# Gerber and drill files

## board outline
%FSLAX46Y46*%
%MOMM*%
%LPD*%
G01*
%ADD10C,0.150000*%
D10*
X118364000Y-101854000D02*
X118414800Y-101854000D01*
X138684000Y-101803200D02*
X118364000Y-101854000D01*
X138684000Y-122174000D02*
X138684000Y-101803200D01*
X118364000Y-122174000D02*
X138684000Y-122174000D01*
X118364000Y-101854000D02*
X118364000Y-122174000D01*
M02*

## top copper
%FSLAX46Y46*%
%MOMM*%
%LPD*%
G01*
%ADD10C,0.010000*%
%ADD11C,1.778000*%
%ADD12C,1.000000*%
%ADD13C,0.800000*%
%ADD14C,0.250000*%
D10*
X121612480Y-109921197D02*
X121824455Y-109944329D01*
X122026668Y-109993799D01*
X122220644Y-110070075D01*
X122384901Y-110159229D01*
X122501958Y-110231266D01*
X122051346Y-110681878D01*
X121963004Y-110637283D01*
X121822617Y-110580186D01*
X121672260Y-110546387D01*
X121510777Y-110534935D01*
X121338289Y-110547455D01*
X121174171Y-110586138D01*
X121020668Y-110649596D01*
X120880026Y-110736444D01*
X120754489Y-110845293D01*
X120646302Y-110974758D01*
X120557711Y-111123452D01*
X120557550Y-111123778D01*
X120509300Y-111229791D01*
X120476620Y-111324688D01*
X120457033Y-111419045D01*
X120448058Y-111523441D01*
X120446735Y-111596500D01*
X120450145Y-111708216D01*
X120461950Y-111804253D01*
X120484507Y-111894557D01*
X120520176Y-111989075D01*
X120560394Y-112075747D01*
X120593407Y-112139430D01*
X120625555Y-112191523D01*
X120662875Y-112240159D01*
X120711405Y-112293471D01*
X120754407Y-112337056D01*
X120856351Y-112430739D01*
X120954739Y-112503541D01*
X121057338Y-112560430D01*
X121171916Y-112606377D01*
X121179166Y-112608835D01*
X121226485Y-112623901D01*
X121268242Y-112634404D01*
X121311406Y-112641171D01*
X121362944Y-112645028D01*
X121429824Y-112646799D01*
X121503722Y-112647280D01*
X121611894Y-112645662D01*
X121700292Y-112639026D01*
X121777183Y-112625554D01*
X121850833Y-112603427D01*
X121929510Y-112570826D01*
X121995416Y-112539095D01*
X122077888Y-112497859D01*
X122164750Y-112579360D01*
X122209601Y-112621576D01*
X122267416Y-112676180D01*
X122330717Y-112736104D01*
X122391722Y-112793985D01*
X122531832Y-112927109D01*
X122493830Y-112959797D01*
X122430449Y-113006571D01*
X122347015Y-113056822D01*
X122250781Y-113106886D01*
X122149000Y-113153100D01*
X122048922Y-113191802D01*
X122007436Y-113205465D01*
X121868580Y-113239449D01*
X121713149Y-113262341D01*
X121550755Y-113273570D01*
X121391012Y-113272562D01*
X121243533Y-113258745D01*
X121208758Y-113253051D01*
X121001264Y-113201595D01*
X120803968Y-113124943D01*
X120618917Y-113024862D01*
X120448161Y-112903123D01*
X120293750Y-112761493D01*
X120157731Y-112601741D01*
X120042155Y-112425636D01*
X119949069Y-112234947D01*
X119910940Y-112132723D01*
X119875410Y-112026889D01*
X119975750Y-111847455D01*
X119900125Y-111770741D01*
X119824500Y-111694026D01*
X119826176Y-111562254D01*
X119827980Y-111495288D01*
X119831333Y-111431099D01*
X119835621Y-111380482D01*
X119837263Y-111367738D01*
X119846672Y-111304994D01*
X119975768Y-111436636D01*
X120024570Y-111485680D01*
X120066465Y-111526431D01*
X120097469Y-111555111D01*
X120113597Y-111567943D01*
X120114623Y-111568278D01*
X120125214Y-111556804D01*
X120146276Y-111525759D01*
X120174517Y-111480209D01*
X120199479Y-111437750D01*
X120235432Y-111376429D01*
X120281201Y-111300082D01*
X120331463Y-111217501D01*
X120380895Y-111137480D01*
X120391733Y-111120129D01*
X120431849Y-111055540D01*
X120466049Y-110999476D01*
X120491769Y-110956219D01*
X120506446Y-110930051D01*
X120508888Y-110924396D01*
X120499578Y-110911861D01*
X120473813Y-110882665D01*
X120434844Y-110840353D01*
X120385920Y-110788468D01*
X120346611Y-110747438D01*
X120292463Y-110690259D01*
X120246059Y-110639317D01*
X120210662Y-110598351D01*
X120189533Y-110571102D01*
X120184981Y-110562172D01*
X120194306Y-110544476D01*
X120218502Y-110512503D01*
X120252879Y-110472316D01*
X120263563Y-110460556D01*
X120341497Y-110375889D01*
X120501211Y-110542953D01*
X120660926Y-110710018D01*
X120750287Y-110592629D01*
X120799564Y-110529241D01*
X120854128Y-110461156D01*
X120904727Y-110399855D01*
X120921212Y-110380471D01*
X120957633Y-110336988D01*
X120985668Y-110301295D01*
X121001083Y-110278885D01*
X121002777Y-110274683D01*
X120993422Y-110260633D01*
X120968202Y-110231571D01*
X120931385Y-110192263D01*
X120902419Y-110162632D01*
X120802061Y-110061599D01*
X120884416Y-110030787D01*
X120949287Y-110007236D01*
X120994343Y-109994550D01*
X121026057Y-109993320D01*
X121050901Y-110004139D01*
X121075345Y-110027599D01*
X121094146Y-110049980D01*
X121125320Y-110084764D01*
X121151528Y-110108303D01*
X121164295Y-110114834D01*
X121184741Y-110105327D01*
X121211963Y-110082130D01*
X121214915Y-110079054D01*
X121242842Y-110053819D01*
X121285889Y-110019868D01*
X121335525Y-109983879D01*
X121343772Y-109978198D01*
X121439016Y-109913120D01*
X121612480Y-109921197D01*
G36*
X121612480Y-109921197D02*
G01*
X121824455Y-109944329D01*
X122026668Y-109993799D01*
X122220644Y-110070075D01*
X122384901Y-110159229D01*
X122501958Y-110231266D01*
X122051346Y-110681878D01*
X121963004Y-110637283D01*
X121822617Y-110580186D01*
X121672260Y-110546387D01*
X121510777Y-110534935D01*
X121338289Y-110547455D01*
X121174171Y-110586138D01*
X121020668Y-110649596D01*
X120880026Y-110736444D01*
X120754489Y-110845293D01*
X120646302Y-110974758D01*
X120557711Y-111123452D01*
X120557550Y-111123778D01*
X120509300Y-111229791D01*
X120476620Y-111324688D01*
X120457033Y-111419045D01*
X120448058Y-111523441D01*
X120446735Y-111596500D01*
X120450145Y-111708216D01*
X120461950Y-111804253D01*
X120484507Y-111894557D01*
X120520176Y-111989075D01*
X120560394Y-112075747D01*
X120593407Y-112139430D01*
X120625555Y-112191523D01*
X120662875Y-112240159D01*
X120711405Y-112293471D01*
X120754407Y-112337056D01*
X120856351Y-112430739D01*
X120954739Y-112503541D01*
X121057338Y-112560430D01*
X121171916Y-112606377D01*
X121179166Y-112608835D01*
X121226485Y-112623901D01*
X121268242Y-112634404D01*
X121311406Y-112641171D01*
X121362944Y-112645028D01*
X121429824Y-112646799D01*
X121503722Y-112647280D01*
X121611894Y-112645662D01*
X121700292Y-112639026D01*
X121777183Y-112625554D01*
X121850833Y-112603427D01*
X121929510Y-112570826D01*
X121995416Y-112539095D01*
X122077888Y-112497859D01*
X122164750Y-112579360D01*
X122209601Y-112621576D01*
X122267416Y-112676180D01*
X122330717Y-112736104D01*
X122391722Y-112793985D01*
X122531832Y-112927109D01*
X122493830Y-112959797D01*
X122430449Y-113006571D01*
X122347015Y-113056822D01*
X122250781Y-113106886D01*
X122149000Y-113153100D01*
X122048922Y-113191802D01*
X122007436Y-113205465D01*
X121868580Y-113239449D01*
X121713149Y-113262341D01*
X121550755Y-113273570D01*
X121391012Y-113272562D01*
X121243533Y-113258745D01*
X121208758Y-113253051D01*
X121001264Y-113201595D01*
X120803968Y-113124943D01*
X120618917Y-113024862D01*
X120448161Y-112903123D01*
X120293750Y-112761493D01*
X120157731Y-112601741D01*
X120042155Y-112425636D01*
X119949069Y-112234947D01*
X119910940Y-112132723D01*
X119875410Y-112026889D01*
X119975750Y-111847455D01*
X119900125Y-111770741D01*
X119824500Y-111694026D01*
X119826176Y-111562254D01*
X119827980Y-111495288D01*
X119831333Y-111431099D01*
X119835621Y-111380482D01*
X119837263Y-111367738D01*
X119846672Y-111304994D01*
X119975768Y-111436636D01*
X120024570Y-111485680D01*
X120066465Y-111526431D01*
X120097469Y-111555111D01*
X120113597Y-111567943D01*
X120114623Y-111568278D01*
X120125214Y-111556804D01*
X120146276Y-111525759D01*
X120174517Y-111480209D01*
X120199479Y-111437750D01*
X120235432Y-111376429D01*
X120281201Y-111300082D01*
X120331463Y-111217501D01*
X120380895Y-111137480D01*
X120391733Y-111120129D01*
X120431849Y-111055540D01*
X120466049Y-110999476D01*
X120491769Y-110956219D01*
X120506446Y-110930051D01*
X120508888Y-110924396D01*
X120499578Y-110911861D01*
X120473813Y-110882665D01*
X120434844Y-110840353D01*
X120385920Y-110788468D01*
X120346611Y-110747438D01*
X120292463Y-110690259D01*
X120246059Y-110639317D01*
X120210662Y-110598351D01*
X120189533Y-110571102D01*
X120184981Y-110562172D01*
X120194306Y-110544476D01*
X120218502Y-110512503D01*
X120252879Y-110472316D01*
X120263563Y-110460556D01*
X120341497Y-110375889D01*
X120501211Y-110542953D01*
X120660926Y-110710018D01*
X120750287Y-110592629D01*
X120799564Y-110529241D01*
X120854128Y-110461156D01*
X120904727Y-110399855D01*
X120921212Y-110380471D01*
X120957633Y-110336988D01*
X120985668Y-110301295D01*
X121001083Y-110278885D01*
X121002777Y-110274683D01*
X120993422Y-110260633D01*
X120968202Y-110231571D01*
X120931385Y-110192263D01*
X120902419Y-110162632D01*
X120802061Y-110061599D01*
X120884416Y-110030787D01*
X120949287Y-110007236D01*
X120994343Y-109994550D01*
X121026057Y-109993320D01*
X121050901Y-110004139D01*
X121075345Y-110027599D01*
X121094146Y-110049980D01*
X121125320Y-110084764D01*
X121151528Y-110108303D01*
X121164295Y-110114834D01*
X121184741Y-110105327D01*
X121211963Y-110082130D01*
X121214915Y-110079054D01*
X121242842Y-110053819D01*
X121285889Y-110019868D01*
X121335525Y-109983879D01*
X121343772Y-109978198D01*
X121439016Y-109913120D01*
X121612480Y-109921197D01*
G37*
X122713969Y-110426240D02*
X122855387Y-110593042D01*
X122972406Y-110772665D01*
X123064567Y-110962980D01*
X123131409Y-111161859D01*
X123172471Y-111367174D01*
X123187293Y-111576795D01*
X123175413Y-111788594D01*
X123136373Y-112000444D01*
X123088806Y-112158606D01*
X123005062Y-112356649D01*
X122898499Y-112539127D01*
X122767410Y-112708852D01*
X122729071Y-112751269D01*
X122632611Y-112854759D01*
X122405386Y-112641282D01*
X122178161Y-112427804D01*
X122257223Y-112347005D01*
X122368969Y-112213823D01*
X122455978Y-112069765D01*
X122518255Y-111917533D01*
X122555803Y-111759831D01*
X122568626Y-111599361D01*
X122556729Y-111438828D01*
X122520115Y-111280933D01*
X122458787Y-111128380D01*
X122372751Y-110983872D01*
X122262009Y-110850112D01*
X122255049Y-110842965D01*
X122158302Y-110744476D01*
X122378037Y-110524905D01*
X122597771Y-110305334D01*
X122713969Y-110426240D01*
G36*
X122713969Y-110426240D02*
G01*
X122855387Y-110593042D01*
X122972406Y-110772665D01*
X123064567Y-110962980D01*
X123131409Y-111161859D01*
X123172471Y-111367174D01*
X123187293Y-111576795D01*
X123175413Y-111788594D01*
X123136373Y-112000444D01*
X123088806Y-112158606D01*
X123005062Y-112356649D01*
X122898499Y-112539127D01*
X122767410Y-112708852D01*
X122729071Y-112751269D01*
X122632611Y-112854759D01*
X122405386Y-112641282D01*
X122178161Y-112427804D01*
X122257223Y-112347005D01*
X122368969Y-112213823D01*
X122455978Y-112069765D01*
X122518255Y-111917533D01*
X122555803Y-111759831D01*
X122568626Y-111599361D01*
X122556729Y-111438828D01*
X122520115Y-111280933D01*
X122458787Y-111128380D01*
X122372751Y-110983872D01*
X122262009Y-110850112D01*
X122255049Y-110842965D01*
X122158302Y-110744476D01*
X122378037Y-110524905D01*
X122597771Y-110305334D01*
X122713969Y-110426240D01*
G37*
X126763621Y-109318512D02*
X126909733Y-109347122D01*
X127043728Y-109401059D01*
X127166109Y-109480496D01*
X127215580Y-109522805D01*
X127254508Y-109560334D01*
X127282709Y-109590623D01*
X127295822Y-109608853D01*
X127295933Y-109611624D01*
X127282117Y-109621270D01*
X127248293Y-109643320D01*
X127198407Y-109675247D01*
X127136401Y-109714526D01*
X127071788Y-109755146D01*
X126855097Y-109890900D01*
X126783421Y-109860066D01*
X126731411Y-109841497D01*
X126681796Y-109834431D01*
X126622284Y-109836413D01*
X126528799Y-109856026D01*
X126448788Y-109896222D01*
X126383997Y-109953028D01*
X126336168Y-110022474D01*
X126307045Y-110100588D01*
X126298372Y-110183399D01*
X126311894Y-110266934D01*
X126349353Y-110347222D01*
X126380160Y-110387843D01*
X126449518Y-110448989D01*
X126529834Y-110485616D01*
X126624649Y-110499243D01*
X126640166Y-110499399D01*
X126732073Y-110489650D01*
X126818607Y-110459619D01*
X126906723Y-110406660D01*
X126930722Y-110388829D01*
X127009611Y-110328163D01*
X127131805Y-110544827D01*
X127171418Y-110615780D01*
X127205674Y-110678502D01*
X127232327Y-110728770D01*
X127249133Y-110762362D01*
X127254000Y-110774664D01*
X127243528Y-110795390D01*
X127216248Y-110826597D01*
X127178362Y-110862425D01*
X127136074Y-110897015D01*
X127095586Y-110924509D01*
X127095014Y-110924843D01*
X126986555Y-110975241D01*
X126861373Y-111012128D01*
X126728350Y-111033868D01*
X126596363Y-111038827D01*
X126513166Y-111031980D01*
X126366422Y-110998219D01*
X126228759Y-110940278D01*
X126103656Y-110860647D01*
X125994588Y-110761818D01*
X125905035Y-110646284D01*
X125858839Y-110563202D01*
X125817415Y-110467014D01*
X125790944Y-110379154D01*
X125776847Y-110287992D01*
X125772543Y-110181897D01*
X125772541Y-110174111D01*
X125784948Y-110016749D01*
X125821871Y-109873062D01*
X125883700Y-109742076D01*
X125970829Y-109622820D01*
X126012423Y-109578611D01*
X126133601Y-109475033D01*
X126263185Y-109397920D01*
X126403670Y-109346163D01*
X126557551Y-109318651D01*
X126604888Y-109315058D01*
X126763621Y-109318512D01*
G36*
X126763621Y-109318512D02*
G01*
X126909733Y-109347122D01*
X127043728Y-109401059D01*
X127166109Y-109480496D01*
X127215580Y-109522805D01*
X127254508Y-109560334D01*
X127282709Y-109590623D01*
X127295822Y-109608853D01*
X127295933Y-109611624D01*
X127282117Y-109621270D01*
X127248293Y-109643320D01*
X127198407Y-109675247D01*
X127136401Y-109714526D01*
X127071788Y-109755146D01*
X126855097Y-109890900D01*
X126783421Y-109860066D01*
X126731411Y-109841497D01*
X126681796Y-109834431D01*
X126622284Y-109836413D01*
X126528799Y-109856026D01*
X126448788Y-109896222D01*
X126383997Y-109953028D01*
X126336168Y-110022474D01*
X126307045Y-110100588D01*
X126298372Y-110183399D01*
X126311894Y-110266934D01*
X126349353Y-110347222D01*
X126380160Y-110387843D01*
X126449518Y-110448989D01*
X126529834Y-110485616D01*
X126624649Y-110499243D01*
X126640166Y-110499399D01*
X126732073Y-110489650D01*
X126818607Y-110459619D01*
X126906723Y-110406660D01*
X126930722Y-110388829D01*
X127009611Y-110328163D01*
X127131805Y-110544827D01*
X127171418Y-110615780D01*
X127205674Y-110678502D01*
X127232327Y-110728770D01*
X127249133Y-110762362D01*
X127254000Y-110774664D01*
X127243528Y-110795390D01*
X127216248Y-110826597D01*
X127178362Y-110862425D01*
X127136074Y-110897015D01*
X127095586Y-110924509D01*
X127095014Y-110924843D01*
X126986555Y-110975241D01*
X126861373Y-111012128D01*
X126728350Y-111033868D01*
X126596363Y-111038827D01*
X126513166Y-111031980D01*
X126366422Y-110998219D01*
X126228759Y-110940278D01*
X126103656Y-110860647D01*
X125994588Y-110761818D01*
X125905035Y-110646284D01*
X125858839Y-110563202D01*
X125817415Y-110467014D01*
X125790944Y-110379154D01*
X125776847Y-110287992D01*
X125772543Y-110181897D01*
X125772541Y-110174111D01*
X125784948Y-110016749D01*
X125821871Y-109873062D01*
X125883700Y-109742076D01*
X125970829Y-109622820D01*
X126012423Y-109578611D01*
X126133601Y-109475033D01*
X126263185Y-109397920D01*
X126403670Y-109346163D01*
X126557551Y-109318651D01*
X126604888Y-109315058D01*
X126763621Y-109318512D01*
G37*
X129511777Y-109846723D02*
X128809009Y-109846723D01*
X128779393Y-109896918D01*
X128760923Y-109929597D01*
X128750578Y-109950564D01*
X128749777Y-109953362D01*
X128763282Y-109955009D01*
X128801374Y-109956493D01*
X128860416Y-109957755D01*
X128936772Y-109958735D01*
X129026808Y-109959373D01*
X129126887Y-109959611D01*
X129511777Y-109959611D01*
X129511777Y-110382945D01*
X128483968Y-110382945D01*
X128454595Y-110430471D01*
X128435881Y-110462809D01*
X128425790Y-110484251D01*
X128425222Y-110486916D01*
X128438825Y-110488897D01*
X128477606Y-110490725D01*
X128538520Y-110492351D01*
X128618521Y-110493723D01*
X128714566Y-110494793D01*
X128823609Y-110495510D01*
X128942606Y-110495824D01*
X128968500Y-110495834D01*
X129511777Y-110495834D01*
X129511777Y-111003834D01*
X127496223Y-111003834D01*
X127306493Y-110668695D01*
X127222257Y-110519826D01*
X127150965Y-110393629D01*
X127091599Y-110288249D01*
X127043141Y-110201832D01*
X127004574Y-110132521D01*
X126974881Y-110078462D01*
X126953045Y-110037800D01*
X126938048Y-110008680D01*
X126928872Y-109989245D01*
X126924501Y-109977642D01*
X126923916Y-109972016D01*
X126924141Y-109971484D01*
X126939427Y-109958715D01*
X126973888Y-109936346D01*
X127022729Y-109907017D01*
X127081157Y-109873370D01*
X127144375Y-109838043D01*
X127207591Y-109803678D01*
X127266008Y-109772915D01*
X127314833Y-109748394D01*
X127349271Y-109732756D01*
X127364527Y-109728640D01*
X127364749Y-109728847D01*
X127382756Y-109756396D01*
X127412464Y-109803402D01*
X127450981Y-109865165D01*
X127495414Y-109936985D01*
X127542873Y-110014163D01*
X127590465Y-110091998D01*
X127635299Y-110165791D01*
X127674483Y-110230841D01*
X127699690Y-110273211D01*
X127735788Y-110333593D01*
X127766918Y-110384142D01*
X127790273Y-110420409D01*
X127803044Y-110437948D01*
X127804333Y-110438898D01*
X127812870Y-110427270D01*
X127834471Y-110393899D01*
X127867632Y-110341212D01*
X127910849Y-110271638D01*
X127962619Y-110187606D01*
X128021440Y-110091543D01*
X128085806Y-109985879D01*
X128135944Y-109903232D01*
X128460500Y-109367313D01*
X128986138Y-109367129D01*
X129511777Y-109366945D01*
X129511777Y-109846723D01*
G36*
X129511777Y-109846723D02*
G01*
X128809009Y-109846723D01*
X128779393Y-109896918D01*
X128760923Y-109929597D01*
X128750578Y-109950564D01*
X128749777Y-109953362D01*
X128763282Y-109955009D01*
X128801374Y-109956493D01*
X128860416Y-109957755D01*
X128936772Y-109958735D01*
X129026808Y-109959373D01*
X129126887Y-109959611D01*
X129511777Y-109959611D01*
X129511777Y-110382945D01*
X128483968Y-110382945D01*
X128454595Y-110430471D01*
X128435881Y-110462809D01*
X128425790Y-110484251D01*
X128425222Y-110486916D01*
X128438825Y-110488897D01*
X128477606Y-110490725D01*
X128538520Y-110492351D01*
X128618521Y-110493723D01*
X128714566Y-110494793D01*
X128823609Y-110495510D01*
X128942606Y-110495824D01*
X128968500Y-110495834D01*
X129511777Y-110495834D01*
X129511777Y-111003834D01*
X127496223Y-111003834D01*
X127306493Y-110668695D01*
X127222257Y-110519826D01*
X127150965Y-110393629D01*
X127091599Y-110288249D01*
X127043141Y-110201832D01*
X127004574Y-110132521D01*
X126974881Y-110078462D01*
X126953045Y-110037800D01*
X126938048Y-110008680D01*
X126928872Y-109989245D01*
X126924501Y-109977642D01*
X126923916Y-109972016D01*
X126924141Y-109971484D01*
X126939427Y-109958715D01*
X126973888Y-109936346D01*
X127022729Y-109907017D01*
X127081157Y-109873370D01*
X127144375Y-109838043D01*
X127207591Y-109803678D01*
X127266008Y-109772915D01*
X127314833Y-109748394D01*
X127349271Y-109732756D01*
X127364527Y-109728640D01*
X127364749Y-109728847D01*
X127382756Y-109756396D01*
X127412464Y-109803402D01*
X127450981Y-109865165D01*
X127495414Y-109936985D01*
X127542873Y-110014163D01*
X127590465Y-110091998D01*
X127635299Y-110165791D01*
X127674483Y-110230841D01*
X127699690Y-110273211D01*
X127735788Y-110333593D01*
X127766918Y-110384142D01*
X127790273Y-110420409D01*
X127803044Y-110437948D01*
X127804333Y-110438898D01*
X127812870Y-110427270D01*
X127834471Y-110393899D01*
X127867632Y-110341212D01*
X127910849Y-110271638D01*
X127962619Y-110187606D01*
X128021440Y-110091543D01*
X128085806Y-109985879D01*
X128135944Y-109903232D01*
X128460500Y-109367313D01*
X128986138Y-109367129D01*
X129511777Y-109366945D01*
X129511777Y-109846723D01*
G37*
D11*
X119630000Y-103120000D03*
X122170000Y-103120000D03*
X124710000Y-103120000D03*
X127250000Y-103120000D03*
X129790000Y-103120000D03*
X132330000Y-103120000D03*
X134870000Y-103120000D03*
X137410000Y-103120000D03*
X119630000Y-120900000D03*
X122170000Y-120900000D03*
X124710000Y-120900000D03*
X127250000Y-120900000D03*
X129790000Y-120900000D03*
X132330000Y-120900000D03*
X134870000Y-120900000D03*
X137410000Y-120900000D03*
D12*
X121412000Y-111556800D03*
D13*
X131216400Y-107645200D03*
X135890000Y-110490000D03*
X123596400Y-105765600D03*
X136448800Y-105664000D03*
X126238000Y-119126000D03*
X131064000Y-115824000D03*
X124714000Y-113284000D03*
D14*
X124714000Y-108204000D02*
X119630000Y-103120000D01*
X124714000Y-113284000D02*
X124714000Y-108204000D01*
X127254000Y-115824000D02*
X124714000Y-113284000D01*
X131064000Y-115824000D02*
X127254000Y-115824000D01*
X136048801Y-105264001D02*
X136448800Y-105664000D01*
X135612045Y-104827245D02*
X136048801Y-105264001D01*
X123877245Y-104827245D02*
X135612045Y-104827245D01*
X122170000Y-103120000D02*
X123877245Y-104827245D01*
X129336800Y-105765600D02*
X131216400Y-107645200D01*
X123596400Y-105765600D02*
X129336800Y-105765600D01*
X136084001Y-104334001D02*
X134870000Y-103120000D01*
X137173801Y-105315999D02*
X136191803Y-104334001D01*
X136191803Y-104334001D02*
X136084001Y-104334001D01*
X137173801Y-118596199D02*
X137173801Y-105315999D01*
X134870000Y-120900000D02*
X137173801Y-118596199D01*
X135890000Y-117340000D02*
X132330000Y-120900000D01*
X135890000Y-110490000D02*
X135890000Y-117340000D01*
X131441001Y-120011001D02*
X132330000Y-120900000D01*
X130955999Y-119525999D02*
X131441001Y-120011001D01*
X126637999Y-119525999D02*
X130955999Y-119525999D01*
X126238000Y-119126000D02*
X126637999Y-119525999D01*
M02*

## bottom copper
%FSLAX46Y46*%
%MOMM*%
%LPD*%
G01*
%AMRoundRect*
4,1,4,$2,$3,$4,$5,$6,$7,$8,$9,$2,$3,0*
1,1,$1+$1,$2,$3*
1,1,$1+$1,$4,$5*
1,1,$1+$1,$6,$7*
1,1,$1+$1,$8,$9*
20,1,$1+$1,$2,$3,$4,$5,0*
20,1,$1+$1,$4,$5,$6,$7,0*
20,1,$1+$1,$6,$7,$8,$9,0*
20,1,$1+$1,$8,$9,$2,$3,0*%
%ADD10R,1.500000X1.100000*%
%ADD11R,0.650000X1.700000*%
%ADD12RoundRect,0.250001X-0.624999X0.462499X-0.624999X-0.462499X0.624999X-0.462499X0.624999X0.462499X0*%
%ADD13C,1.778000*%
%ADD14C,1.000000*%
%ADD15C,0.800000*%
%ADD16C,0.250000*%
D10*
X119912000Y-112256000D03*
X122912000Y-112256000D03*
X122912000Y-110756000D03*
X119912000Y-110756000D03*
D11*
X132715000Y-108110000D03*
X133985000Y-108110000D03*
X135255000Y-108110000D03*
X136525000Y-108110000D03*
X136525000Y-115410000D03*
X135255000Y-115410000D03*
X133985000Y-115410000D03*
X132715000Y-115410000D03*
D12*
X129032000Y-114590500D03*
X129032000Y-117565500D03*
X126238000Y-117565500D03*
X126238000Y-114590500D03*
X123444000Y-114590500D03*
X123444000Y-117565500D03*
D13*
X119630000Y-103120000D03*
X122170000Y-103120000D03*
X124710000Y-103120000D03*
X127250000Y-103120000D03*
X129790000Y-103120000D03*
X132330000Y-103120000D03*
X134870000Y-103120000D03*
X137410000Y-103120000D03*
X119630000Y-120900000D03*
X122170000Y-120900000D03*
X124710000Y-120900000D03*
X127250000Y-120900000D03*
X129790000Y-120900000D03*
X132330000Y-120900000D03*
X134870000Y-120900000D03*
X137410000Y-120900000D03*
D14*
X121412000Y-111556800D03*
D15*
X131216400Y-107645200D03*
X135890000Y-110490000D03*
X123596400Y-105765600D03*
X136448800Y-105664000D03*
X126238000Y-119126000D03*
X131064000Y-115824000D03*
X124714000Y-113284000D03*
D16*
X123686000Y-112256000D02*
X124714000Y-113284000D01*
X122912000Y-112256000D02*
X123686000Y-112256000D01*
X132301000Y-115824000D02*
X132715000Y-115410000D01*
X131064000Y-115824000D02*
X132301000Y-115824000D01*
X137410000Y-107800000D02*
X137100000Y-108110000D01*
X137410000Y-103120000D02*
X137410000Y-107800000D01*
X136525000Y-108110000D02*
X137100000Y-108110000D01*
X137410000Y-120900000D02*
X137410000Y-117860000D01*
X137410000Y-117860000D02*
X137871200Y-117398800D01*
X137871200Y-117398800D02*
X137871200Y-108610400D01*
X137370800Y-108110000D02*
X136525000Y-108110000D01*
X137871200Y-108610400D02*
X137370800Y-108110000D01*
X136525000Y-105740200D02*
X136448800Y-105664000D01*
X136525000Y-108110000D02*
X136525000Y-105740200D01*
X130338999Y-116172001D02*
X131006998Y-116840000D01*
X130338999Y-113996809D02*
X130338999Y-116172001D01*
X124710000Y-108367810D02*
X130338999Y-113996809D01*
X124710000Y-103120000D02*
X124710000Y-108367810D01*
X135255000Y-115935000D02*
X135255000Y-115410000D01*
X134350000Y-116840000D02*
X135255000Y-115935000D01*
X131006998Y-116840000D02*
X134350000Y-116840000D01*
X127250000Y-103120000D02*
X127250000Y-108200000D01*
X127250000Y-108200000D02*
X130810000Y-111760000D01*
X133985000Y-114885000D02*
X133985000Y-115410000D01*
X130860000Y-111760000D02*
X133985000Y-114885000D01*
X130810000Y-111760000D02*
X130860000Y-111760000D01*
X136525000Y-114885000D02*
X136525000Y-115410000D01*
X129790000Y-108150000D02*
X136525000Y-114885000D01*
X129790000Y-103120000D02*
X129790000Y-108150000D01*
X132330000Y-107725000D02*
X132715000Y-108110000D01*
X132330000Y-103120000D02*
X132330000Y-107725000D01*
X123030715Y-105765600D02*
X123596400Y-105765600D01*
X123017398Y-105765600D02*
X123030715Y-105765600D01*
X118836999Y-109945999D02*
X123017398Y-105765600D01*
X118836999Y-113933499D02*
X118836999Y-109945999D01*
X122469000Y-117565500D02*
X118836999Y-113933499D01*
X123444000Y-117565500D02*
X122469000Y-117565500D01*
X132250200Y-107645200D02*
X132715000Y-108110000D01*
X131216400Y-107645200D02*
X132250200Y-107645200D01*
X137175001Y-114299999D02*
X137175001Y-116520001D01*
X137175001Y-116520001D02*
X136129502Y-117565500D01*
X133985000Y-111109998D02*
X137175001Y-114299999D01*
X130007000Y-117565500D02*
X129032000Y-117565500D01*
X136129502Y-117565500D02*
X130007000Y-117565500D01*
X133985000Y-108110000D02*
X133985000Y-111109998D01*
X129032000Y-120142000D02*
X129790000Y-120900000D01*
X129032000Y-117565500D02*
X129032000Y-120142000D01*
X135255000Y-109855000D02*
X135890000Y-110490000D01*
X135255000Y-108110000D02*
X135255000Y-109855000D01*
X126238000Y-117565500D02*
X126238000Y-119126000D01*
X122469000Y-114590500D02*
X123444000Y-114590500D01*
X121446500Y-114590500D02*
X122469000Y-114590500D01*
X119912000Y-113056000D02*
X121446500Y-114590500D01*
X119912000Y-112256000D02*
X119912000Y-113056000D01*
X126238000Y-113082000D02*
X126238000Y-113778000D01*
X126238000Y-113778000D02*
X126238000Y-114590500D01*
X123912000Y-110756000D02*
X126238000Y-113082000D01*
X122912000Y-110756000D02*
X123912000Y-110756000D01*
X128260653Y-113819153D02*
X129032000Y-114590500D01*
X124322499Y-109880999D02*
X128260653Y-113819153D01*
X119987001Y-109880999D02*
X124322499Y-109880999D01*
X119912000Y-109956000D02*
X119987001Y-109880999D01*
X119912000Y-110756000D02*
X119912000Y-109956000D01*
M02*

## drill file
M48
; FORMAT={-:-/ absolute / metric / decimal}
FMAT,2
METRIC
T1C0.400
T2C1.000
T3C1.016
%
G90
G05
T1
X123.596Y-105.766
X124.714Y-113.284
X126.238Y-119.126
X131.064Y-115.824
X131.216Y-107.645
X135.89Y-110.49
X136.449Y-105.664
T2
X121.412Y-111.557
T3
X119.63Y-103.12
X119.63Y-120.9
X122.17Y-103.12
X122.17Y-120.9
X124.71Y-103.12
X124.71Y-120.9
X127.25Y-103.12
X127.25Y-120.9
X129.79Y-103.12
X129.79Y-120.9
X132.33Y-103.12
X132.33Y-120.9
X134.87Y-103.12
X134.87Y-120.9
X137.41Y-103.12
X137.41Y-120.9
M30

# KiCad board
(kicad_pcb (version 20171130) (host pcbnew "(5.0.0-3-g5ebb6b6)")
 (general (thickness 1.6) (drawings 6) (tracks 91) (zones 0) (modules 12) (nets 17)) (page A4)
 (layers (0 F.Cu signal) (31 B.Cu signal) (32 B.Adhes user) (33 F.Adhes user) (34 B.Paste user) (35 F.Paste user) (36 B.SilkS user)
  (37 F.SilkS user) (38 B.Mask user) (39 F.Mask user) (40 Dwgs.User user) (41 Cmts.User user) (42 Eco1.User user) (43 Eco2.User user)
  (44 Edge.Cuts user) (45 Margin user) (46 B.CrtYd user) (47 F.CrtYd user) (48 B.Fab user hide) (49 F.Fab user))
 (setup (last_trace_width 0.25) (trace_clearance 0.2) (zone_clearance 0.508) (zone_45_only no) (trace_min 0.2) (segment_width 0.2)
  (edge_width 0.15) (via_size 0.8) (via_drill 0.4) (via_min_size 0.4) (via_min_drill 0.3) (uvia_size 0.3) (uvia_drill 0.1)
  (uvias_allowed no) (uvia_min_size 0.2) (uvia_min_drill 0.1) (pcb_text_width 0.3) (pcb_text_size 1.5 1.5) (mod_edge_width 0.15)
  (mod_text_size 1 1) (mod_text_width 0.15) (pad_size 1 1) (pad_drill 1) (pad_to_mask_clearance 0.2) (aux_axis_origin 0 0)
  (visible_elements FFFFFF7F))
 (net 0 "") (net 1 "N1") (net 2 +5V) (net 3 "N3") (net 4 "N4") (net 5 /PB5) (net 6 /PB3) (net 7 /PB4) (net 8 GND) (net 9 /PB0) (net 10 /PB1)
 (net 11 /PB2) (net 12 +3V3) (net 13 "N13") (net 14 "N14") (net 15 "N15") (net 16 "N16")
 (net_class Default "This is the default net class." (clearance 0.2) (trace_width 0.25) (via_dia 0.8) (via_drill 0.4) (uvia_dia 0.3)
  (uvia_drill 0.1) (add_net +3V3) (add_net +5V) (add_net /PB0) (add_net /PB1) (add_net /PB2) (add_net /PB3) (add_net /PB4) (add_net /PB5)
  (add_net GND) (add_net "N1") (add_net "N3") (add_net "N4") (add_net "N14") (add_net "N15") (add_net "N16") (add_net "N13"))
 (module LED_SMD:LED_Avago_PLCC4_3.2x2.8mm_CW (layer B.Cu) (at 121.412 111.506)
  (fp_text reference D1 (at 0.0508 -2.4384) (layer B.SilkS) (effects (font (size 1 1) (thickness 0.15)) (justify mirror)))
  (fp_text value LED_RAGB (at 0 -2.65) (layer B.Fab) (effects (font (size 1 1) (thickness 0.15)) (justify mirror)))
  (pad 1 smd rect (at -1.5 0.75) (size 1.5 1.1) (layers B.Cu B.Paste B.Mask) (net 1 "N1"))
  (pad 2 smd rect (at 1.5 0.75) (size 1.5 1.1) (layers B.Cu B.Paste B.Mask) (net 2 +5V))
  (pad 3 smd rect (at 1.5 -0.75) (size 1.5 1.1) (layers B.Cu B.Paste B.Mask) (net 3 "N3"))
  (pad 4 smd rect (at -1.5 -0.75) (size 1.5 1.1) (layers B.Cu B.Paste B.Mask) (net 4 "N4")))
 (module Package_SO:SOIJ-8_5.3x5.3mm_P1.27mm (layer B.Cu) (at 134.62 111.76 270)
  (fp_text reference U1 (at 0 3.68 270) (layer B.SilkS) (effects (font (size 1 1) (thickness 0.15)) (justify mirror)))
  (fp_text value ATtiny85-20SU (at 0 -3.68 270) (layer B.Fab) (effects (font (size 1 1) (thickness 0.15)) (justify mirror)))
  (pad 1 smd rect (at -3.65 1.905 270) (size 1.7 0.65) (layers B.Cu B.Paste B.Mask) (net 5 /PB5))
  (pad 2 smd rect (at -3.65 0.635 270) (size 1.7 0.65) (layers B.Cu B.Paste B.Mask) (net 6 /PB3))
  (pad 3 smd rect (at -3.65 -0.635 270) (size 1.7 0.65) (layers B.Cu B.Paste B.Mask) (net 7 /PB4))
  (pad 4 smd rect (at -3.65 -1.905 270) (size 1.7 0.65) (layers B.Cu B.Paste B.Mask) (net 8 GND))
  (pad 5 smd rect (at 3.65 -1.905 270) (size 1.7 0.65) (layers B.Cu B.Paste B.Mask) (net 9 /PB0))
  (pad 6 smd rect (at 3.65 -0.635 270) (size 1.7 0.65) (layers B.Cu B.Paste B.Mask) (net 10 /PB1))
  (pad 7 smd rect (at 3.65 0.635 270) (size 1.7 0.65) (layers B.Cu B.Paste B.Mask) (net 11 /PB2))
  (pad 8 smd rect (at 3.65 1.905 270) (size 1.7 0.65) (layers B.Cu B.Paste B.Mask) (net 2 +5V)))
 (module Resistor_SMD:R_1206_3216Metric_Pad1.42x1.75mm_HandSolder (layer B.Cu) (at 129.032 116.078 270)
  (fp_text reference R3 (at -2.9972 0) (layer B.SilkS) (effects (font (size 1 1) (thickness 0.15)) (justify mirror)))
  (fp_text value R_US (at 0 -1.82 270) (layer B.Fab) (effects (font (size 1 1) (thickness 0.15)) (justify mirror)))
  (pad 1 smd roundrect (at -1.4875 0 270) (size 1.425 1.75) (layers B.Cu B.Paste B.Mask) (roundrect_rratio 0.175439) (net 4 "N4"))
  (pad 2 smd roundrect (at 1.4875 0 270) (size 1.425 1.75) (layers B.Cu B.Paste B.Mask) (roundrect_rratio 0.175439) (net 6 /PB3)))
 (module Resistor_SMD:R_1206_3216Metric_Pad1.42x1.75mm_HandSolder (layer B.Cu) (at 126.238 116.078 270)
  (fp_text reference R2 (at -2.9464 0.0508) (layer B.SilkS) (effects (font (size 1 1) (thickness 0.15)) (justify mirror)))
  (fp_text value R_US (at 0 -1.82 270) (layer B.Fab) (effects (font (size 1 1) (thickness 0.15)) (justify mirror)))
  (pad 2 smd roundrect (at 1.4875 0 270) (size 1.425 1.75) (layers B.Cu B.Paste B.Mask) (roundrect_rratio 0.175439) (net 7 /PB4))
  (pad 1 smd roundrect (at -1.4875 0 270) (size 1.425 1.75) (layers B.Cu B.Paste B.Mask) (roundrect_rratio 0.175439) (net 3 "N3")))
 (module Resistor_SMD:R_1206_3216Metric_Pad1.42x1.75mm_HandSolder (layer B.Cu) (at 123.444 116.078 270)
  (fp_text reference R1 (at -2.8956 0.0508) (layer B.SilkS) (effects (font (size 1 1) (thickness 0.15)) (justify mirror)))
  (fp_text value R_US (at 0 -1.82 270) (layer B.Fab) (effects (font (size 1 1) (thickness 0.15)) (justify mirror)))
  (pad 1 smd roundrect (at -1.4875 0 270) (size 1.425 1.75) (layers B.Cu B.Paste B.Mask) (roundrect_rratio 0.175439) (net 1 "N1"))
  (pad 2 smd roundrect (at 1.4875 0 270) (size 1.425 1.75) (layers B.Cu B.Paste B.Mask) (roundrect_rratio 0.175439) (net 5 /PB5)))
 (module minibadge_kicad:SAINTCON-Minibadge (layer F.Cu) (at 118.36 101.85)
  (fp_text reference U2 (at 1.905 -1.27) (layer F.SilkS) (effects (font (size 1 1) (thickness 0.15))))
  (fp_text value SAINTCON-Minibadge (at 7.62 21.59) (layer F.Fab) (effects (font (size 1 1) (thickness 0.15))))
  (pad 1 thru_hole circle (at 1.27 1.27 90) (size 1.778 1.778) (drill 1.016) (layers *.Cu *.Mask) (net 2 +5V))
  (pad 2 thru_hole circle (at 3.81 1.27 90) (size 1.778 1.778) (drill 1.016) (layers *.Cu *.Mask) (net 8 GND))
  (pad 3 thru_hole circle (at 6.35 1.27 90) (size 1.778 1.778) (drill 1.016) (layers *.Cu *.Mask) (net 10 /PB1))
  (pad 4 thru_hole circle (at 8.89 1.27 90) (size 1.778 1.778) (drill 1.016) (layers *.Cu *.Mask) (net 11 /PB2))
  (pad 5 thru_hole circle (at 11.43 1.27 90) (size 1.778 1.778) (drill 1.016) (layers *.Cu *.Mask) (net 9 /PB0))
  (pad 6 thru_hole circle (at 13.97 1.27 90) (size 1.778 1.778) (drill 1.016) (layers *.Cu *.Mask) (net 5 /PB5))
  (pad 7 thru_hole circle (at 16.51 1.27 90) (size 1.778 1.778) (drill 1.016) (layers *.Cu *.Mask) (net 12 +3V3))
  (pad 8 thru_hole circle (at 19.05 1.27 90) (size 1.778 1.778) (drill 1.016) (layers *.Cu *.Mask) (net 8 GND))
  (pad 9 thru_hole circle (at 1.27 19.05 90) (size 1.778 1.778) (drill 1.016) (layers *.Cu *.Mask) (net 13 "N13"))
  (pad 10 thru_hole circle (at 3.81 19.05 90) (size 1.778 1.778) (drill 1.016) (layers *.Cu *.Mask) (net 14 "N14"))
  (pad 11 thru_hole circle (at 6.35 19.05 90) (size 1.778 1.778) (drill 1.016) (layers *.Cu *.Mask) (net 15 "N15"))
  (pad 12 thru_hole circle (at 8.89 19.05 90) (size 1.778 1.778) (drill 1.016) (layers *.Cu *.Mask) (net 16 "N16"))
  (pad 13 thru_hole circle (at 11.43 19.05 90) (size 1.778 1.778) (drill 1.016) (layers *.Cu *.Mask) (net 6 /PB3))
  (pad 14 thru_hole circle (at 13.97 19.05 90) (size 1.778 1.778) (drill 1.016) (layers *.Cu *.Mask) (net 7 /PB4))
  (pad 15 thru_hole circle (at 16.51 19.05 90) (size 1.778 1.778) (drill 1.016) (layers *.Cu *.Mask) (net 12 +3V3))
  (pad 16 thru_hole circle (at 19.05 19.05 90) (size 1.778 1.778) (drill 1.016) (layers *.Cu *.Mask) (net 8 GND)))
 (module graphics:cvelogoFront (layer F.Cu) (at 128.27 111.9775)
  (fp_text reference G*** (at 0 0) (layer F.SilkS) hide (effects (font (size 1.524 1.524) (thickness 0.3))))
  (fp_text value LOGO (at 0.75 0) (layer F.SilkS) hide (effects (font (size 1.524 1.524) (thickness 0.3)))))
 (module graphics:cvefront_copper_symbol (layer F.Cu) (at 128.27 111.9775)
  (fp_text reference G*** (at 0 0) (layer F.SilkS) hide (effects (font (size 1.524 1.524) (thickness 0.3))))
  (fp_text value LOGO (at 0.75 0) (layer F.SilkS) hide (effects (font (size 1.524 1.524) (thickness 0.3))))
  (fp_poly
   (pts (xy -6.65752 -2.056303) (xy -6.445545 -2.033171) (xy -6.243332 -1.983701) (xy -6.049356 -1.907425) (xy -5.885099 -1.818271)
    (xy -5.768042 -1.746234) (xy -6.218654 -1.295622) (xy -6.306996 -1.340217) (xy -6.447383 -1.397314) (xy -6.59774 -1.431113)
    (xy -6.759223 -1.442565) (xy -6.931711 -1.430045) (xy -7.095829 -1.391362) (xy -7.249332 -1.327904) (xy -7.389974 -1.241056)
    (xy -7.515511 -1.132207) (xy -7.623698 -1.002742) (xy -7.712289 -0.854048) (xy -7.71245 -0.853722) (xy -7.7607 -0.747709)
    (xy -7.79338 -0.652812) (xy -7.812967 -0.558455) (xy -7.821942 -0.454059) (xy -7.823265 -0.381) (xy -7.819855 -0.269284)
    (xy -7.80805 -0.173247) (xy -7.785493 -0.082943) (xy -7.749824 0.011575) (xy -7.709606 0.098247) (xy -7.676593 0.16193)
    (xy -7.644445 0.214023) (xy -7.607125 0.262659) (xy -7.558595 0.315971) (xy -7.515593 0.359556) (xy -7.413649 0.453239)
    (xy -7.315261 0.526041) (xy -7.212662 0.58293) (xy -7.098084 0.628877) (xy -7.090834 0.631335) (xy -7.043515 0.646401)
    (xy -7.001758 0.656904) (xy -6.958594 0.663671) (xy -6.907056 0.667528) (xy -6.840176 0.669299) (xy -6.766278 0.66978)
    (xy -6.658106 0.668162) (xy -6.569708 0.661526) (xy -6.492817 0.648054) (xy -6.419167 0.625927) (xy -6.34049 0.593326)
    (xy -6.274584 0.561595) (xy -6.192112 0.520359) (xy -6.10525 0.60186) (xy -6.060399 0.644076) (xy -6.002584 0.69868)
    (xy -5.939283 0.758604) (xy -5.878278 0.816485) (xy -5.738168 0.949609) (xy -5.77617 0.982297) (xy -5.839551 1.029071)
    (xy -5.922985 1.079322) (xy -6.019219 1.129386) (xy -6.121 1.1756) (xy -6.221078 1.214302) (xy -6.262564 1.227965)
    (xy -6.40142 1.261949) (xy -6.556851 1.284841) (xy -6.719245 1.29607) (xy -6.878988 1.295062) (xy -7.026467 1.281245)
    (xy -7.061242 1.275551) (xy -7.268736 1.224095) (xy -7.466032 1.147443) (xy -7.651083 1.047362) (xy -7.821839 0.925623)
    (xy -7.97625 0.783993) (xy -8.112269 0.624241) (xy -8.227845 0.448136) (xy -8.320931 0.257447) (xy -8.35906 0.155223)
    (xy -8.39459 0.049389) (xy -8.29425 -0.130045) (xy -8.369875 -0.206759) (xy -8.4455 -0.283474) (xy -8.443824 -0.415246)
    (xy -8.44202 -0.482212) (xy -8.438667 -0.546401) (xy -8.434379 -0.597018) (xy -8.432737 -0.609762) (xy -8.423328 -0.672506)
    (xy -8.294232 -0.540864) (xy -8.24543 -0.49182) (xy -8.203535 -0.451069) (xy -8.172531 -0.422389) (xy -8.156403 -0.409557)
    (xy -8.155377 -0.409222) (xy -8.144786 -0.420696) (xy -8.123724 -0.451741) (xy -8.095483 -0.497291) (xy -8.070521 -0.53975)
    (xy -8.034568 -0.601071) (xy -7.988799 -0.677418) (xy -7.938537 -0.759999) (xy -7.889105 -0.84002) (xy -7.878267 -0.857371)
    (xy -7.838151 -0.92196) (xy -7.803951 -0.978024) (xy -7.778231 -1.021281) (xy -7.763554 -1.047449) (xy -7.761112 -1.053104)
    (xy -7.770422 -1.065639) (xy -7.796187 -1.094835) (xy -7.835156 -1.137147) (xy -7.88408 -1.189032) (xy -7.923389 -1.230062)
    (xy -7.977537 -1.287241) (xy -8.023941 -1.338183) (xy -8.059338 -1.379149) (xy -8.080467 -1.406398) (xy -8.085019 -1.415328)
    (xy -8.075694 -1.433024) (xy -8.051498 -1.464997) (xy -8.017121 -1.505184) (xy -8.006437 -1.516944) (xy -7.928503 -1.601611)
    (xy -7.768789 -1.434547) (xy -7.609074 -1.267482) (xy -7.519713 -1.384871) (xy -7.470436 -1.448259) (xy -7.415872 -1.516344)
    (xy -7.365273 -1.577645) (xy -7.348788 -1.597029) (xy -7.312367 -1.640512) (xy -7.284332 -1.676205) (xy -7.268917 -1.698615)
    (xy -7.267223 -1.702817) (xy -7.276578 -1.716867) (xy -7.301798 -1.745929) (xy -7.338615 -1.785237) (xy -7.367581 -1.814868)
    (xy -7.467939 -1.915901) (xy -7.385584 -1.946713) (xy -7.320713 -1.970264) (xy -7.275657 -1.98295) (xy -7.243943 -1.98418)
    (xy -7.219099 -1.973361) (xy -7.194655 -1.949901) (xy -7.175854 -1.92752) (xy -7.14468 -1.892736) (xy -7.118472 -1.869197)
    (xy -7.105705 -1.862666) (xy -7.085259 -1.872173) (xy -7.058037 -1.89537) (xy -7.055085 -1.898446) (xy -7.027158 -1.923681)
    (xy -6.984111 -1.957632) (xy -6.934475 -1.993621) (xy -6.926228 -1.999302) (xy -6.830984 -2.06438) (xy -6.65752 -2.056303))
   (layer F.Cu) (width 0.01))
  (fp_poly
   (pts (xy -5.556031 -1.55126) (xy -5.414613 -1.384458) (xy -5.297594 -1.204835) (xy -5.205433 -1.01452) (xy -5.138591 -0.815641)
    (xy -5.097529 -0.610326) (xy -5.082707 -0.400705) (xy -5.094587 -0.188906) (xy -5.133627 0.022944) (xy -5.181194 0.181106)
    (xy -5.264938 0.379149) (xy -5.371501 0.561627) (xy -5.50259 0.731352) (xy -5.540929 0.773769) (xy -5.637389 0.877259)
    (xy -5.864614 0.663782) (xy -6.091839 0.450304) (xy -6.012777 0.369505) (xy -5.901031 0.236323) (xy -5.814022 0.092265)
    (xy -5.751745 -0.059967) (xy -5.714197 -0.217669) (xy -5.701374 -0.378139) (xy -5.713271 -0.538672) (xy -5.749885 -0.696567)
    (xy -5.811213 -0.84912) (xy -5.897249 -0.993628) (xy -6.007991 -1.127388) (xy -6.014951 -1.134535) (xy -6.111698 -1.233024)
    (xy -5.891963 -1.452595) (xy -5.672229 -1.672166) (xy -5.556031 -1.55126))
   (layer F.Cu) (width 0.01)))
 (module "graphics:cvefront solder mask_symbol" (layer F.Cu) (at 128.27 111.9775)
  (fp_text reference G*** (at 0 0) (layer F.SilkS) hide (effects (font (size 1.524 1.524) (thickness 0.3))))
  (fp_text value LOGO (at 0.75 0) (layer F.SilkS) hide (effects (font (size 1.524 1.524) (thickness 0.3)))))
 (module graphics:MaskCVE (layer F.Cu) (at 128.27 111.9775)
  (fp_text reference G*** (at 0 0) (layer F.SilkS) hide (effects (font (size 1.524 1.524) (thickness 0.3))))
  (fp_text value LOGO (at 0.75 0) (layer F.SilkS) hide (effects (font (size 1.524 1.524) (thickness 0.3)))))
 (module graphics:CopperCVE (layer F.Cu) (at 128.27 111.9775)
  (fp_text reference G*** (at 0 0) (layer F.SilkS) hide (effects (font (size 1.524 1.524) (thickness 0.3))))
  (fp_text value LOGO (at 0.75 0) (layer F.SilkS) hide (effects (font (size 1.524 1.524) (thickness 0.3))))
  (fp_poly
   (pts (xy -1.506379 -2.658988) (xy -1.360267 -2.630378) (xy -1.226272 -2.576441) (xy -1.103891 -2.497004) (xy -1.05442 -2.454695)
    (xy -1.015492 -2.417166) (xy -0.987291 -2.386877) (xy -0.974178 -2.368647) (xy -0.974067 -2.365876) (xy -0.987883 -2.35623)
    (xy -1.021707 -2.33418) (xy -1.071593 -2.302253) (xy -1.133599 -2.262974) (xy -1.198212 -2.222354) (xy -1.414903 -2.0866)
    (xy -1.486579 -2.117434) (xy -1.538589 -2.136003) (xy -1.588204 -2.143069) (xy -1.647716 -2.141087) (xy -1.741201 -2.121474)
    (xy -1.821212 -2.081278) (xy -1.886003 -2.024472) (xy -1.933832 -1.955026) (xy -1.962955 -1.876912) (xy -1.971628 -1.794101)
    (xy -1.958106 -1.710566) (xy -1.920647 -1.630278) (xy -1.88984 -1.589657) (xy -1.820482 -1.528511) (xy -1.740166 -1.491884)
    (xy -1.645351 -1.478257) (xy -1.629834 -1.478101) (xy -1.537927 -1.48785) (xy -1.451393 -1.517881) (xy -1.363277 -1.57084)
    (xy -1.339278 -1.588671) (xy -1.260389 -1.649337) (xy -1.138195 -1.432673) (xy -1.098582 -1.36172) (xy -1.064326 -1.298998)
    (xy -1.037673 -1.24873) (xy -1.020867 -1.215138) (xy -1.016 -1.202836) (xy -1.026472 -1.18211) (xy -1.053752 -1.150903)
    (xy -1.091638 -1.115075) (xy -1.133926 -1.080485) (xy -1.174414 -1.052991) (xy -1.174986 -1.052657) (xy -1.283445 -1.002259)
    (xy -1.408627 -0.965372) (xy -1.54165 -0.943632) (xy -1.673637 -0.938673) (xy -1.756834 -0.94552) (xy -1.903578 -0.979281)
    (xy -2.041241 -1.037222) (xy -2.166344 -1.116853) (xy -2.275412 -1.215682) (xy -2.364965 -1.331216) (xy -2.411161 -1.414298)
    (xy -2.452585 -1.510486) (xy -2.479056 -1.598346) (xy -2.493153 -1.689508) (xy -2.497457 -1.795603) (xy -2.497459 -1.803389)
    (xy -2.485052 -1.960751) (xy -2.448129 -2.104438) (xy -2.3863 -2.235424) (xy -2.299171 -2.35468) (xy -2.257577 -2.398889)
    (xy -2.136399 -2.502467) (xy -2.006815 -2.57958) (xy -1.86633 -2.631337) (xy -1.712449 -2.658849) (xy -1.665112 -2.662442)
    (xy -1.506379 -2.658988))
   (layer F.Cu) (width 0.01))
  (fp_poly
   (pts (xy 1.241777 -2.130777) (xy 0.539009 -2.130777) (xy 0.509393 -2.080582) (xy 0.490923 -2.047903) (xy 0.480578 -2.026936)
    (xy 0.479777 -2.024138) (xy 0.493282 -2.022491) (xy 0.531374 -2.021007) (xy 0.590416 -2.019745) (xy 0.666772 -2.018765)
    (xy 0.756808 -2.018127) (xy 0.856887 -2.017889) (xy 1.241777 -2.017889) (xy 1.241777 -1.594555) (xy 0.213968 -1.594555)
    (xy 0.184595 -1.547029) (xy 0.165881 -1.514691) (xy 0.15579 -1.493249) (xy 0.155222 -1.490584) (xy 0.168825 -1.488603)
    (xy 0.207606 -1.486775) (xy 0.26852 -1.485149) (xy 0.348521 -1.483777) (xy 0.444566 -1.482707) (xy 0.553609 -1.48199)
    (xy 0.672606 -1.481676) (xy 0.6985 -1.481666) (xy 1.241777 -1.481666) (xy 1.241777 -0.973666) (xy -0.773777 -0.973666)
    (xy -0.963507 -1.308805) (xy -1.047743 -1.457674) (xy -1.119035 -1.583871) (xy -1.178401 -1.689251) (xy -1.226859 -1.775668)
    (xy -1.265426 -1.844979) (xy -1.295119 -1.899038) (xy -1.316955 -1.9397) (xy -1.331952 -1.96882) (xy -1.341128 -1.988255)
    (xy -1.345499 -1.999858) (xy -1.346084 -2.005484) (xy -1.345859 -2.006016) (xy -1.330573 -2.018785) (xy -1.296112 -2.041154)
    (xy -1.247271 -2.070483) (xy -1.188843 -2.10413) (xy -1.125625 -2.139457) (xy -1.062409 -2.173822) (xy -1.003992 -2.204585)
    (xy -0.955167 -2.229106) (xy -0.920729 -2.244744) (xy -0.905473 -2.24886) (xy -0.905251 -2.248653) (xy -0.887244 -2.221104)
    (xy -0.857536 -2.174098) (xy -0.819019 -2.112335) (xy -0.774586 -2.040515) (xy -0.727127 -1.963337) (xy -0.679535 -1.885502)
    (xy -0.634701 -1.811709) (xy -0.595517 -1.746659) (xy -0.57031 -1.704289) (xy -0.534212 -1.643907) (xy -0.503082 -1.593358)
    (xy -0.479727 -1.557091) (xy -0.466956 -1.539552) (xy -0.465667 -1.538602) (xy -0.45713 -1.55023) (xy -0.435529 -1.583601)
    (xy -0.402368 -1.636288) (xy -0.359151 -1.705862) (xy -0.307381 -1.789894) (xy -0.24856 -1.885957) (xy -0.184194 -1.991621)
    (xy -0.134056 -2.074268) (xy 0.1905 -2.610187) (xy 0.716138 -2.610371) (xy 1.241777 -2.610555) (xy 1.241777 -2.130777))
   (layer F.Cu) (width 0.01)))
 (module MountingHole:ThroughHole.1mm (layer F.Cu) (at 121.412 111.5568)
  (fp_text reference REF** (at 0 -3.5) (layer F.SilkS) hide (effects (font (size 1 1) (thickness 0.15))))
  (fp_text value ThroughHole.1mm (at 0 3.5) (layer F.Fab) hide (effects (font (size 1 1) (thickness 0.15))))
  (pad 1 thru_hole circle (at 0 0) (size 1 1) (drill 1) (layers *.Cu)))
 (gr_line (start 118.364 101.854) (end 118.4148 101.854) (layer Edge.Cuts) (width 0.15))
 (gr_line (start 138.684 101.8032) (end 118.364 101.854) (layer Edge.Cuts) (width 0.15))
 (gr_line (start 138.684 122.174) (end 138.684 101.8032) (layer Edge.Cuts) (width 0.15))
 (gr_line (start 118.364 122.174) (end 138.684 122.174) (layer Edge.Cuts) (width 0.15))
 (gr_line (start 118.364 101.854) (end 118.364 122.174) (layer Edge.Cuts) (width 0.15))
 (via micro (at 131.2164 107.6452) (size 0.8) (drill 0.4) (layers F.Cu B.Cu) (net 5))
 (via micro (at 135.89 110.49) (size 0.8) (drill 0.4) (layers F.Cu B.Cu) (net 7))
 (via micro (at 123.5964 105.7656) (size 0.8) (drill 0.4) (layers F.Cu B.Cu) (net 5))
 (via micro (at 136.4488 105.664) (size 0.8) (drill 0.4) (layers F.Cu B.Cu) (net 8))
 (via micro (at 126.238 119.126) (size 0.8) (drill 0.4) (layers F.Cu B.Cu) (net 7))
 (via micro (at 131.064 115.824) (size 0.8) (drill 0.4) (layers F.Cu B.Cu) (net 2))
 (via micro (at 124.714 113.284) (size 0.8) (drill 0.4) (layers F.Cu B.Cu) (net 2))
 (segment (start 123.686 112.256) (end 124.714 113.284) (width 0.25) (layer B.Cu) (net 2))
 (segment (start 122.912 112.256) (end 123.686 112.256) (width 0.25) (layer B.Cu) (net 2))
 (segment (start 124.714 108.204) (end 119.63 103.12) (width 0.25) (layer F.Cu) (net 2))
 (segment (start 124.714 113.284) (end 124.714 108.204) (width 0.25) (layer F.Cu) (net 2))
 (segment (start 127.254 115.824) (end 124.714 113.284) (width 0.25) (layer F.Cu) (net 2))
 (segment (start 131.064 115.824) (end 127.254 115.824) (width 0.25) (layer F.Cu) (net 2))
 (segment (start 132.301 115.824) (end 132.715 115.41) (width 0.25) (layer B.Cu) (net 2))
 (segment (start 131.064 115.824) (end 132.301 115.824) (width 0.25) (layer B.Cu) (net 2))
 (segment (start 137.41 107.8) (end 137.1 108.11) (width 0.25) (layer B.Cu) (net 8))
 (segment (start 137.41 103.12) (end 137.41 107.8) (width 0.25) (layer B.Cu) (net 8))
 (segment (start 136.525 108.11) (end 137.1 108.11) (width 0.25) (layer B.Cu) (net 8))
 (segment (start 137.41 120.9) (end 137.41 117.86) (width 0.25) (layer B.Cu) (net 8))
 (segment (start 137.41 117.86) (end 137.8712 117.3988) (width 0.25) (layer B.Cu) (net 8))
 (segment (start 137.8712 117.3988) (end 137.8712 108.6104) (width 0.25) (layer B.Cu) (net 8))
 (segment (start 137.3708 108.11) (end 136.525 108.11) (width 0.25) (layer B.Cu) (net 8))
 (segment (start 137.8712 108.6104) (end 137.3708 108.11) (width 0.25) (layer B.Cu) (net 8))
 (segment (start 136.525 105.7402) (end 136.4488 105.664) (width 0.25) (layer B.Cu) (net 8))
 (segment (start 136.525 108.11) (end 136.525 105.7402) (width 0.25) (layer B.Cu) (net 8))
 (segment (start 136.048801 105.264001) (end 136.4488 105.664) (width 0.25) (layer F.Cu) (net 8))
 (segment (start 135.612045 104.827245) (end 136.048801 105.264001) (width 0.25) (layer F.Cu) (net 8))
 (segment (start 123.877245 104.827245) (end 135.612045 104.827245) (width 0.25) (layer F.Cu) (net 8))
 (segment (start 122.17 103.12) (end 123.877245 104.827245) (width 0.25) (layer F.Cu) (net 8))
 (segment (start 130.338999 116.172001) (end 131.006998 116.84) (width 0.25) (layer B.Cu) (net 10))
 (segment (start 130.338999 113.996809) (end 130.338999 116.172001) (width 0.25) (layer B.Cu) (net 10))
 (segment (start 124.71 108.36781) (end 130.338999 113.996809) (width 0.25) (layer B.Cu) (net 10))
 (segment (start 124.71 103.12) (end 124.71 108.36781) (width 0.25) (layer B.Cu) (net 10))
 (segment (start 135.255 115.935) (end 135.255 115.41) (width 0.25) (layer B.Cu) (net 10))
 (segment (start 134.35 116.84) (end 135.255 115.935) (width 0.25) (layer B.Cu) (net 10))
 (segment (start 131.006998 116.84) (end 134.35 116.84) (width 0.25) (layer B.Cu) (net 10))
 (segment (start 127.25 103.12) (end 127.25 108.2) (width 0.25) (layer B.Cu) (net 11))
 (segment (start 127.25 108.2) (end 130.81 111.76) (width 0.25) (layer B.Cu) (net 11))
 (segment (start 133.985 114.885) (end 133.985 115.41) (width 0.25) (layer B.Cu) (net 11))
 (segment (start 130.86 111.76) (end 133.985 114.885) (width 0.25) (layer B.Cu) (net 11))
 (segment (start 130.81 111.76) (end 130.86 111.76) (width 0.25) (layer B.Cu) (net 11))
 (segment (start 136.525 114.885) (end 136.525 115.41) (width 0.25) (layer B.Cu) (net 9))
 (segment (start 129.79 108.15) (end 136.525 114.885) (width 0.25) (layer B.Cu) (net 9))
 (segment (start 129.79 103.12) (end 129.79 108.15) (width 0.25) (layer B.Cu) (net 9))
 (segment (start 132.33 107.725) (end 132.715 108.11) (width 0.25) (layer B.Cu) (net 5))
 (segment (start 132.33 103.12) (end 132.33 107.725) (width 0.25) (layer B.Cu) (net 5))
 (segment (start 123.030715 105.7656) (end 123.5964 105.7656) (width 0.25) (layer B.Cu) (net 5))
 (segment (start 123.017398 105.7656) (end 123.030715 105.7656) (width 0.25) (layer B.Cu) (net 5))
 (segment (start 118.836999 109.945999) (end 123.017398 105.7656) (width 0.25) (layer B.Cu) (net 5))
 (segment (start 118.836999 113.933499) (end 118.836999 109.945999) (width 0.25) (layer B.Cu) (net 5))
 (segment (start 122.469 117.5655) (end 118.836999 113.933499) (width 0.25) (layer B.Cu) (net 5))
 (segment (start 123.444 117.5655) (end 122.469 117.5655) (width 0.25) (layer B.Cu) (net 5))
 (segment (start 129.3368 105.7656) (end 131.2164 107.6452) (width 0.25) (layer F.Cu) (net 5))
 (segment (start 123.5964 105.7656) (end 129.3368 105.7656) (width 0.25) (layer F.Cu) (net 5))
 (segment (start 132.2502 107.6452) (end 132.715 108.11) (width 0.25) (layer B.Cu) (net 5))
 (segment (start 131.2164 107.6452) (end 132.2502 107.6452) (width 0.25) (layer B.Cu) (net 5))
 (segment (start 136.084001 104.334001) (end 134.87 103.12) (width 0.25) (layer F.Cu) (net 12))
 (segment (start 137.173801 105.315999) (end 136.191803 104.334001) (width 0.25) (layer F.Cu) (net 12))
 (segment (start 136.191803 104.334001) (end 136.084001 104.334001) (width 0.25) (layer F.Cu) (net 12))
 (segment (start 137.173801 118.596199) (end 137.173801 105.315999) (width 0.25) (layer F.Cu) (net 12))
 (segment (start 134.87 120.9) (end 137.173801 118.596199) (width 0.25) (layer F.Cu) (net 12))
 (segment (start 137.175001 114.299999) (end 137.175001 116.520001) (width 0.25) (layer B.Cu) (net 6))
 (segment (start 137.175001 116.520001) (end 136.129502 117.5655) (width 0.25) (layer B.Cu) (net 6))
 (segment (start 133.985 111.109998) (end 137.175001 114.299999) (width 0.25) (layer B.Cu) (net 6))
 (segment (start 130.007 117.5655) (end 129.032 117.5655) (width 0.25) (layer B.Cu) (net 6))
 (segment (start 136.129502 117.5655) (end 130.007 117.5655) (width 0.25) (layer B.Cu) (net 6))
 (segment (start 133.985 108.11) (end 133.985 111.109998) (width 0.25) (layer B.Cu) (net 6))
 (segment (start 129.032 120.142) (end 129.79 120.9) (width 0.25) (layer B.Cu) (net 6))
 (segment (start 129.032 117.5655) (end 129.032 120.142) (width 0.25) (layer B.Cu) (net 6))
 (segment (start 135.255 109.855) (end 135.89 110.49) (width 0.25) (layer B.Cu) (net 7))
 (segment (start 135.255 108.11) (end 135.255 109.855) (width 0.25) (layer B.Cu) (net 7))
 (segment (start 126.238 117.5655) (end 126.238 119.126) (width 0.25) (layer B.Cu) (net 7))
 (segment (start 135.89 117.34) (end 132.33 120.9) (width 0.25) (layer F.Cu) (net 7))
 (segment (start 135.89 110.49) (end 135.89 117.34) (width 0.25) (layer F.Cu) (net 7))
 (segment (start 131.441001 120.011001) (end 132.33 120.9) (width 0.25) (layer F.Cu) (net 7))
 (segment (start 130.955999 119.525999) (end 131.441001 120.011001) (width 0.25) (layer F.Cu) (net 7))
 (segment (start 126.637999 119.525999) (end 130.955999 119.525999) (width 0.25) (layer F.Cu) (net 7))
 (segment (start 126.238 119.126) (end 126.637999 119.525999) (width 0.25) (layer F.Cu) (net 7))
 (segment (start 122.469 114.5905) (end 123.444 114.5905) (width 0.25) (layer B.Cu) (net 1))
 (segment (start 121.4465 114.5905) (end 122.469 114.5905) (width 0.25) (layer B.Cu) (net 1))
 (segment (start 119.912 113.056) (end 121.4465 114.5905) (width 0.25) (layer B.Cu) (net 1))
 (segment (start 119.912 112.256) (end 119.912 113.056) (width 0.25) (layer B.Cu) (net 1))
 (segment (start 126.238 113.082) (end 126.238 113.778) (width 0.25) (layer B.Cu) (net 3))
 (segment (start 126.238 113.778) (end 126.238 114.5905) (width 0.25) (layer B.Cu) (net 3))
 (segment (start 123.912 110.756) (end 126.238 113.082) (width 0.25) (layer B.Cu) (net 3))
 (segment (start 122.912 110.756) (end 123.912 110.756) (width 0.25) (layer B.Cu) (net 3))
 (segment (start 128.260653 113.819153) (end 129.032 114.5905) (width 0.25) (layer B.Cu) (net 4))
 (segment (start 124.322499 109.880999) (end 128.260653 113.819153) (width 0.25) (layer B.Cu) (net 4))
 (segment (start 119.987001 109.880999) (end 124.322499 109.880999) (width 0.25) (layer B.Cu) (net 4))
 (segment (start 119.912 109.956) (end 119.987001 109.880999) (width 0.25) (layer B.Cu) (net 4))
 (segment (start 119.912 110.756) (end 119.912 109.956) (width 0.25) (layer B.Cu) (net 4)))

